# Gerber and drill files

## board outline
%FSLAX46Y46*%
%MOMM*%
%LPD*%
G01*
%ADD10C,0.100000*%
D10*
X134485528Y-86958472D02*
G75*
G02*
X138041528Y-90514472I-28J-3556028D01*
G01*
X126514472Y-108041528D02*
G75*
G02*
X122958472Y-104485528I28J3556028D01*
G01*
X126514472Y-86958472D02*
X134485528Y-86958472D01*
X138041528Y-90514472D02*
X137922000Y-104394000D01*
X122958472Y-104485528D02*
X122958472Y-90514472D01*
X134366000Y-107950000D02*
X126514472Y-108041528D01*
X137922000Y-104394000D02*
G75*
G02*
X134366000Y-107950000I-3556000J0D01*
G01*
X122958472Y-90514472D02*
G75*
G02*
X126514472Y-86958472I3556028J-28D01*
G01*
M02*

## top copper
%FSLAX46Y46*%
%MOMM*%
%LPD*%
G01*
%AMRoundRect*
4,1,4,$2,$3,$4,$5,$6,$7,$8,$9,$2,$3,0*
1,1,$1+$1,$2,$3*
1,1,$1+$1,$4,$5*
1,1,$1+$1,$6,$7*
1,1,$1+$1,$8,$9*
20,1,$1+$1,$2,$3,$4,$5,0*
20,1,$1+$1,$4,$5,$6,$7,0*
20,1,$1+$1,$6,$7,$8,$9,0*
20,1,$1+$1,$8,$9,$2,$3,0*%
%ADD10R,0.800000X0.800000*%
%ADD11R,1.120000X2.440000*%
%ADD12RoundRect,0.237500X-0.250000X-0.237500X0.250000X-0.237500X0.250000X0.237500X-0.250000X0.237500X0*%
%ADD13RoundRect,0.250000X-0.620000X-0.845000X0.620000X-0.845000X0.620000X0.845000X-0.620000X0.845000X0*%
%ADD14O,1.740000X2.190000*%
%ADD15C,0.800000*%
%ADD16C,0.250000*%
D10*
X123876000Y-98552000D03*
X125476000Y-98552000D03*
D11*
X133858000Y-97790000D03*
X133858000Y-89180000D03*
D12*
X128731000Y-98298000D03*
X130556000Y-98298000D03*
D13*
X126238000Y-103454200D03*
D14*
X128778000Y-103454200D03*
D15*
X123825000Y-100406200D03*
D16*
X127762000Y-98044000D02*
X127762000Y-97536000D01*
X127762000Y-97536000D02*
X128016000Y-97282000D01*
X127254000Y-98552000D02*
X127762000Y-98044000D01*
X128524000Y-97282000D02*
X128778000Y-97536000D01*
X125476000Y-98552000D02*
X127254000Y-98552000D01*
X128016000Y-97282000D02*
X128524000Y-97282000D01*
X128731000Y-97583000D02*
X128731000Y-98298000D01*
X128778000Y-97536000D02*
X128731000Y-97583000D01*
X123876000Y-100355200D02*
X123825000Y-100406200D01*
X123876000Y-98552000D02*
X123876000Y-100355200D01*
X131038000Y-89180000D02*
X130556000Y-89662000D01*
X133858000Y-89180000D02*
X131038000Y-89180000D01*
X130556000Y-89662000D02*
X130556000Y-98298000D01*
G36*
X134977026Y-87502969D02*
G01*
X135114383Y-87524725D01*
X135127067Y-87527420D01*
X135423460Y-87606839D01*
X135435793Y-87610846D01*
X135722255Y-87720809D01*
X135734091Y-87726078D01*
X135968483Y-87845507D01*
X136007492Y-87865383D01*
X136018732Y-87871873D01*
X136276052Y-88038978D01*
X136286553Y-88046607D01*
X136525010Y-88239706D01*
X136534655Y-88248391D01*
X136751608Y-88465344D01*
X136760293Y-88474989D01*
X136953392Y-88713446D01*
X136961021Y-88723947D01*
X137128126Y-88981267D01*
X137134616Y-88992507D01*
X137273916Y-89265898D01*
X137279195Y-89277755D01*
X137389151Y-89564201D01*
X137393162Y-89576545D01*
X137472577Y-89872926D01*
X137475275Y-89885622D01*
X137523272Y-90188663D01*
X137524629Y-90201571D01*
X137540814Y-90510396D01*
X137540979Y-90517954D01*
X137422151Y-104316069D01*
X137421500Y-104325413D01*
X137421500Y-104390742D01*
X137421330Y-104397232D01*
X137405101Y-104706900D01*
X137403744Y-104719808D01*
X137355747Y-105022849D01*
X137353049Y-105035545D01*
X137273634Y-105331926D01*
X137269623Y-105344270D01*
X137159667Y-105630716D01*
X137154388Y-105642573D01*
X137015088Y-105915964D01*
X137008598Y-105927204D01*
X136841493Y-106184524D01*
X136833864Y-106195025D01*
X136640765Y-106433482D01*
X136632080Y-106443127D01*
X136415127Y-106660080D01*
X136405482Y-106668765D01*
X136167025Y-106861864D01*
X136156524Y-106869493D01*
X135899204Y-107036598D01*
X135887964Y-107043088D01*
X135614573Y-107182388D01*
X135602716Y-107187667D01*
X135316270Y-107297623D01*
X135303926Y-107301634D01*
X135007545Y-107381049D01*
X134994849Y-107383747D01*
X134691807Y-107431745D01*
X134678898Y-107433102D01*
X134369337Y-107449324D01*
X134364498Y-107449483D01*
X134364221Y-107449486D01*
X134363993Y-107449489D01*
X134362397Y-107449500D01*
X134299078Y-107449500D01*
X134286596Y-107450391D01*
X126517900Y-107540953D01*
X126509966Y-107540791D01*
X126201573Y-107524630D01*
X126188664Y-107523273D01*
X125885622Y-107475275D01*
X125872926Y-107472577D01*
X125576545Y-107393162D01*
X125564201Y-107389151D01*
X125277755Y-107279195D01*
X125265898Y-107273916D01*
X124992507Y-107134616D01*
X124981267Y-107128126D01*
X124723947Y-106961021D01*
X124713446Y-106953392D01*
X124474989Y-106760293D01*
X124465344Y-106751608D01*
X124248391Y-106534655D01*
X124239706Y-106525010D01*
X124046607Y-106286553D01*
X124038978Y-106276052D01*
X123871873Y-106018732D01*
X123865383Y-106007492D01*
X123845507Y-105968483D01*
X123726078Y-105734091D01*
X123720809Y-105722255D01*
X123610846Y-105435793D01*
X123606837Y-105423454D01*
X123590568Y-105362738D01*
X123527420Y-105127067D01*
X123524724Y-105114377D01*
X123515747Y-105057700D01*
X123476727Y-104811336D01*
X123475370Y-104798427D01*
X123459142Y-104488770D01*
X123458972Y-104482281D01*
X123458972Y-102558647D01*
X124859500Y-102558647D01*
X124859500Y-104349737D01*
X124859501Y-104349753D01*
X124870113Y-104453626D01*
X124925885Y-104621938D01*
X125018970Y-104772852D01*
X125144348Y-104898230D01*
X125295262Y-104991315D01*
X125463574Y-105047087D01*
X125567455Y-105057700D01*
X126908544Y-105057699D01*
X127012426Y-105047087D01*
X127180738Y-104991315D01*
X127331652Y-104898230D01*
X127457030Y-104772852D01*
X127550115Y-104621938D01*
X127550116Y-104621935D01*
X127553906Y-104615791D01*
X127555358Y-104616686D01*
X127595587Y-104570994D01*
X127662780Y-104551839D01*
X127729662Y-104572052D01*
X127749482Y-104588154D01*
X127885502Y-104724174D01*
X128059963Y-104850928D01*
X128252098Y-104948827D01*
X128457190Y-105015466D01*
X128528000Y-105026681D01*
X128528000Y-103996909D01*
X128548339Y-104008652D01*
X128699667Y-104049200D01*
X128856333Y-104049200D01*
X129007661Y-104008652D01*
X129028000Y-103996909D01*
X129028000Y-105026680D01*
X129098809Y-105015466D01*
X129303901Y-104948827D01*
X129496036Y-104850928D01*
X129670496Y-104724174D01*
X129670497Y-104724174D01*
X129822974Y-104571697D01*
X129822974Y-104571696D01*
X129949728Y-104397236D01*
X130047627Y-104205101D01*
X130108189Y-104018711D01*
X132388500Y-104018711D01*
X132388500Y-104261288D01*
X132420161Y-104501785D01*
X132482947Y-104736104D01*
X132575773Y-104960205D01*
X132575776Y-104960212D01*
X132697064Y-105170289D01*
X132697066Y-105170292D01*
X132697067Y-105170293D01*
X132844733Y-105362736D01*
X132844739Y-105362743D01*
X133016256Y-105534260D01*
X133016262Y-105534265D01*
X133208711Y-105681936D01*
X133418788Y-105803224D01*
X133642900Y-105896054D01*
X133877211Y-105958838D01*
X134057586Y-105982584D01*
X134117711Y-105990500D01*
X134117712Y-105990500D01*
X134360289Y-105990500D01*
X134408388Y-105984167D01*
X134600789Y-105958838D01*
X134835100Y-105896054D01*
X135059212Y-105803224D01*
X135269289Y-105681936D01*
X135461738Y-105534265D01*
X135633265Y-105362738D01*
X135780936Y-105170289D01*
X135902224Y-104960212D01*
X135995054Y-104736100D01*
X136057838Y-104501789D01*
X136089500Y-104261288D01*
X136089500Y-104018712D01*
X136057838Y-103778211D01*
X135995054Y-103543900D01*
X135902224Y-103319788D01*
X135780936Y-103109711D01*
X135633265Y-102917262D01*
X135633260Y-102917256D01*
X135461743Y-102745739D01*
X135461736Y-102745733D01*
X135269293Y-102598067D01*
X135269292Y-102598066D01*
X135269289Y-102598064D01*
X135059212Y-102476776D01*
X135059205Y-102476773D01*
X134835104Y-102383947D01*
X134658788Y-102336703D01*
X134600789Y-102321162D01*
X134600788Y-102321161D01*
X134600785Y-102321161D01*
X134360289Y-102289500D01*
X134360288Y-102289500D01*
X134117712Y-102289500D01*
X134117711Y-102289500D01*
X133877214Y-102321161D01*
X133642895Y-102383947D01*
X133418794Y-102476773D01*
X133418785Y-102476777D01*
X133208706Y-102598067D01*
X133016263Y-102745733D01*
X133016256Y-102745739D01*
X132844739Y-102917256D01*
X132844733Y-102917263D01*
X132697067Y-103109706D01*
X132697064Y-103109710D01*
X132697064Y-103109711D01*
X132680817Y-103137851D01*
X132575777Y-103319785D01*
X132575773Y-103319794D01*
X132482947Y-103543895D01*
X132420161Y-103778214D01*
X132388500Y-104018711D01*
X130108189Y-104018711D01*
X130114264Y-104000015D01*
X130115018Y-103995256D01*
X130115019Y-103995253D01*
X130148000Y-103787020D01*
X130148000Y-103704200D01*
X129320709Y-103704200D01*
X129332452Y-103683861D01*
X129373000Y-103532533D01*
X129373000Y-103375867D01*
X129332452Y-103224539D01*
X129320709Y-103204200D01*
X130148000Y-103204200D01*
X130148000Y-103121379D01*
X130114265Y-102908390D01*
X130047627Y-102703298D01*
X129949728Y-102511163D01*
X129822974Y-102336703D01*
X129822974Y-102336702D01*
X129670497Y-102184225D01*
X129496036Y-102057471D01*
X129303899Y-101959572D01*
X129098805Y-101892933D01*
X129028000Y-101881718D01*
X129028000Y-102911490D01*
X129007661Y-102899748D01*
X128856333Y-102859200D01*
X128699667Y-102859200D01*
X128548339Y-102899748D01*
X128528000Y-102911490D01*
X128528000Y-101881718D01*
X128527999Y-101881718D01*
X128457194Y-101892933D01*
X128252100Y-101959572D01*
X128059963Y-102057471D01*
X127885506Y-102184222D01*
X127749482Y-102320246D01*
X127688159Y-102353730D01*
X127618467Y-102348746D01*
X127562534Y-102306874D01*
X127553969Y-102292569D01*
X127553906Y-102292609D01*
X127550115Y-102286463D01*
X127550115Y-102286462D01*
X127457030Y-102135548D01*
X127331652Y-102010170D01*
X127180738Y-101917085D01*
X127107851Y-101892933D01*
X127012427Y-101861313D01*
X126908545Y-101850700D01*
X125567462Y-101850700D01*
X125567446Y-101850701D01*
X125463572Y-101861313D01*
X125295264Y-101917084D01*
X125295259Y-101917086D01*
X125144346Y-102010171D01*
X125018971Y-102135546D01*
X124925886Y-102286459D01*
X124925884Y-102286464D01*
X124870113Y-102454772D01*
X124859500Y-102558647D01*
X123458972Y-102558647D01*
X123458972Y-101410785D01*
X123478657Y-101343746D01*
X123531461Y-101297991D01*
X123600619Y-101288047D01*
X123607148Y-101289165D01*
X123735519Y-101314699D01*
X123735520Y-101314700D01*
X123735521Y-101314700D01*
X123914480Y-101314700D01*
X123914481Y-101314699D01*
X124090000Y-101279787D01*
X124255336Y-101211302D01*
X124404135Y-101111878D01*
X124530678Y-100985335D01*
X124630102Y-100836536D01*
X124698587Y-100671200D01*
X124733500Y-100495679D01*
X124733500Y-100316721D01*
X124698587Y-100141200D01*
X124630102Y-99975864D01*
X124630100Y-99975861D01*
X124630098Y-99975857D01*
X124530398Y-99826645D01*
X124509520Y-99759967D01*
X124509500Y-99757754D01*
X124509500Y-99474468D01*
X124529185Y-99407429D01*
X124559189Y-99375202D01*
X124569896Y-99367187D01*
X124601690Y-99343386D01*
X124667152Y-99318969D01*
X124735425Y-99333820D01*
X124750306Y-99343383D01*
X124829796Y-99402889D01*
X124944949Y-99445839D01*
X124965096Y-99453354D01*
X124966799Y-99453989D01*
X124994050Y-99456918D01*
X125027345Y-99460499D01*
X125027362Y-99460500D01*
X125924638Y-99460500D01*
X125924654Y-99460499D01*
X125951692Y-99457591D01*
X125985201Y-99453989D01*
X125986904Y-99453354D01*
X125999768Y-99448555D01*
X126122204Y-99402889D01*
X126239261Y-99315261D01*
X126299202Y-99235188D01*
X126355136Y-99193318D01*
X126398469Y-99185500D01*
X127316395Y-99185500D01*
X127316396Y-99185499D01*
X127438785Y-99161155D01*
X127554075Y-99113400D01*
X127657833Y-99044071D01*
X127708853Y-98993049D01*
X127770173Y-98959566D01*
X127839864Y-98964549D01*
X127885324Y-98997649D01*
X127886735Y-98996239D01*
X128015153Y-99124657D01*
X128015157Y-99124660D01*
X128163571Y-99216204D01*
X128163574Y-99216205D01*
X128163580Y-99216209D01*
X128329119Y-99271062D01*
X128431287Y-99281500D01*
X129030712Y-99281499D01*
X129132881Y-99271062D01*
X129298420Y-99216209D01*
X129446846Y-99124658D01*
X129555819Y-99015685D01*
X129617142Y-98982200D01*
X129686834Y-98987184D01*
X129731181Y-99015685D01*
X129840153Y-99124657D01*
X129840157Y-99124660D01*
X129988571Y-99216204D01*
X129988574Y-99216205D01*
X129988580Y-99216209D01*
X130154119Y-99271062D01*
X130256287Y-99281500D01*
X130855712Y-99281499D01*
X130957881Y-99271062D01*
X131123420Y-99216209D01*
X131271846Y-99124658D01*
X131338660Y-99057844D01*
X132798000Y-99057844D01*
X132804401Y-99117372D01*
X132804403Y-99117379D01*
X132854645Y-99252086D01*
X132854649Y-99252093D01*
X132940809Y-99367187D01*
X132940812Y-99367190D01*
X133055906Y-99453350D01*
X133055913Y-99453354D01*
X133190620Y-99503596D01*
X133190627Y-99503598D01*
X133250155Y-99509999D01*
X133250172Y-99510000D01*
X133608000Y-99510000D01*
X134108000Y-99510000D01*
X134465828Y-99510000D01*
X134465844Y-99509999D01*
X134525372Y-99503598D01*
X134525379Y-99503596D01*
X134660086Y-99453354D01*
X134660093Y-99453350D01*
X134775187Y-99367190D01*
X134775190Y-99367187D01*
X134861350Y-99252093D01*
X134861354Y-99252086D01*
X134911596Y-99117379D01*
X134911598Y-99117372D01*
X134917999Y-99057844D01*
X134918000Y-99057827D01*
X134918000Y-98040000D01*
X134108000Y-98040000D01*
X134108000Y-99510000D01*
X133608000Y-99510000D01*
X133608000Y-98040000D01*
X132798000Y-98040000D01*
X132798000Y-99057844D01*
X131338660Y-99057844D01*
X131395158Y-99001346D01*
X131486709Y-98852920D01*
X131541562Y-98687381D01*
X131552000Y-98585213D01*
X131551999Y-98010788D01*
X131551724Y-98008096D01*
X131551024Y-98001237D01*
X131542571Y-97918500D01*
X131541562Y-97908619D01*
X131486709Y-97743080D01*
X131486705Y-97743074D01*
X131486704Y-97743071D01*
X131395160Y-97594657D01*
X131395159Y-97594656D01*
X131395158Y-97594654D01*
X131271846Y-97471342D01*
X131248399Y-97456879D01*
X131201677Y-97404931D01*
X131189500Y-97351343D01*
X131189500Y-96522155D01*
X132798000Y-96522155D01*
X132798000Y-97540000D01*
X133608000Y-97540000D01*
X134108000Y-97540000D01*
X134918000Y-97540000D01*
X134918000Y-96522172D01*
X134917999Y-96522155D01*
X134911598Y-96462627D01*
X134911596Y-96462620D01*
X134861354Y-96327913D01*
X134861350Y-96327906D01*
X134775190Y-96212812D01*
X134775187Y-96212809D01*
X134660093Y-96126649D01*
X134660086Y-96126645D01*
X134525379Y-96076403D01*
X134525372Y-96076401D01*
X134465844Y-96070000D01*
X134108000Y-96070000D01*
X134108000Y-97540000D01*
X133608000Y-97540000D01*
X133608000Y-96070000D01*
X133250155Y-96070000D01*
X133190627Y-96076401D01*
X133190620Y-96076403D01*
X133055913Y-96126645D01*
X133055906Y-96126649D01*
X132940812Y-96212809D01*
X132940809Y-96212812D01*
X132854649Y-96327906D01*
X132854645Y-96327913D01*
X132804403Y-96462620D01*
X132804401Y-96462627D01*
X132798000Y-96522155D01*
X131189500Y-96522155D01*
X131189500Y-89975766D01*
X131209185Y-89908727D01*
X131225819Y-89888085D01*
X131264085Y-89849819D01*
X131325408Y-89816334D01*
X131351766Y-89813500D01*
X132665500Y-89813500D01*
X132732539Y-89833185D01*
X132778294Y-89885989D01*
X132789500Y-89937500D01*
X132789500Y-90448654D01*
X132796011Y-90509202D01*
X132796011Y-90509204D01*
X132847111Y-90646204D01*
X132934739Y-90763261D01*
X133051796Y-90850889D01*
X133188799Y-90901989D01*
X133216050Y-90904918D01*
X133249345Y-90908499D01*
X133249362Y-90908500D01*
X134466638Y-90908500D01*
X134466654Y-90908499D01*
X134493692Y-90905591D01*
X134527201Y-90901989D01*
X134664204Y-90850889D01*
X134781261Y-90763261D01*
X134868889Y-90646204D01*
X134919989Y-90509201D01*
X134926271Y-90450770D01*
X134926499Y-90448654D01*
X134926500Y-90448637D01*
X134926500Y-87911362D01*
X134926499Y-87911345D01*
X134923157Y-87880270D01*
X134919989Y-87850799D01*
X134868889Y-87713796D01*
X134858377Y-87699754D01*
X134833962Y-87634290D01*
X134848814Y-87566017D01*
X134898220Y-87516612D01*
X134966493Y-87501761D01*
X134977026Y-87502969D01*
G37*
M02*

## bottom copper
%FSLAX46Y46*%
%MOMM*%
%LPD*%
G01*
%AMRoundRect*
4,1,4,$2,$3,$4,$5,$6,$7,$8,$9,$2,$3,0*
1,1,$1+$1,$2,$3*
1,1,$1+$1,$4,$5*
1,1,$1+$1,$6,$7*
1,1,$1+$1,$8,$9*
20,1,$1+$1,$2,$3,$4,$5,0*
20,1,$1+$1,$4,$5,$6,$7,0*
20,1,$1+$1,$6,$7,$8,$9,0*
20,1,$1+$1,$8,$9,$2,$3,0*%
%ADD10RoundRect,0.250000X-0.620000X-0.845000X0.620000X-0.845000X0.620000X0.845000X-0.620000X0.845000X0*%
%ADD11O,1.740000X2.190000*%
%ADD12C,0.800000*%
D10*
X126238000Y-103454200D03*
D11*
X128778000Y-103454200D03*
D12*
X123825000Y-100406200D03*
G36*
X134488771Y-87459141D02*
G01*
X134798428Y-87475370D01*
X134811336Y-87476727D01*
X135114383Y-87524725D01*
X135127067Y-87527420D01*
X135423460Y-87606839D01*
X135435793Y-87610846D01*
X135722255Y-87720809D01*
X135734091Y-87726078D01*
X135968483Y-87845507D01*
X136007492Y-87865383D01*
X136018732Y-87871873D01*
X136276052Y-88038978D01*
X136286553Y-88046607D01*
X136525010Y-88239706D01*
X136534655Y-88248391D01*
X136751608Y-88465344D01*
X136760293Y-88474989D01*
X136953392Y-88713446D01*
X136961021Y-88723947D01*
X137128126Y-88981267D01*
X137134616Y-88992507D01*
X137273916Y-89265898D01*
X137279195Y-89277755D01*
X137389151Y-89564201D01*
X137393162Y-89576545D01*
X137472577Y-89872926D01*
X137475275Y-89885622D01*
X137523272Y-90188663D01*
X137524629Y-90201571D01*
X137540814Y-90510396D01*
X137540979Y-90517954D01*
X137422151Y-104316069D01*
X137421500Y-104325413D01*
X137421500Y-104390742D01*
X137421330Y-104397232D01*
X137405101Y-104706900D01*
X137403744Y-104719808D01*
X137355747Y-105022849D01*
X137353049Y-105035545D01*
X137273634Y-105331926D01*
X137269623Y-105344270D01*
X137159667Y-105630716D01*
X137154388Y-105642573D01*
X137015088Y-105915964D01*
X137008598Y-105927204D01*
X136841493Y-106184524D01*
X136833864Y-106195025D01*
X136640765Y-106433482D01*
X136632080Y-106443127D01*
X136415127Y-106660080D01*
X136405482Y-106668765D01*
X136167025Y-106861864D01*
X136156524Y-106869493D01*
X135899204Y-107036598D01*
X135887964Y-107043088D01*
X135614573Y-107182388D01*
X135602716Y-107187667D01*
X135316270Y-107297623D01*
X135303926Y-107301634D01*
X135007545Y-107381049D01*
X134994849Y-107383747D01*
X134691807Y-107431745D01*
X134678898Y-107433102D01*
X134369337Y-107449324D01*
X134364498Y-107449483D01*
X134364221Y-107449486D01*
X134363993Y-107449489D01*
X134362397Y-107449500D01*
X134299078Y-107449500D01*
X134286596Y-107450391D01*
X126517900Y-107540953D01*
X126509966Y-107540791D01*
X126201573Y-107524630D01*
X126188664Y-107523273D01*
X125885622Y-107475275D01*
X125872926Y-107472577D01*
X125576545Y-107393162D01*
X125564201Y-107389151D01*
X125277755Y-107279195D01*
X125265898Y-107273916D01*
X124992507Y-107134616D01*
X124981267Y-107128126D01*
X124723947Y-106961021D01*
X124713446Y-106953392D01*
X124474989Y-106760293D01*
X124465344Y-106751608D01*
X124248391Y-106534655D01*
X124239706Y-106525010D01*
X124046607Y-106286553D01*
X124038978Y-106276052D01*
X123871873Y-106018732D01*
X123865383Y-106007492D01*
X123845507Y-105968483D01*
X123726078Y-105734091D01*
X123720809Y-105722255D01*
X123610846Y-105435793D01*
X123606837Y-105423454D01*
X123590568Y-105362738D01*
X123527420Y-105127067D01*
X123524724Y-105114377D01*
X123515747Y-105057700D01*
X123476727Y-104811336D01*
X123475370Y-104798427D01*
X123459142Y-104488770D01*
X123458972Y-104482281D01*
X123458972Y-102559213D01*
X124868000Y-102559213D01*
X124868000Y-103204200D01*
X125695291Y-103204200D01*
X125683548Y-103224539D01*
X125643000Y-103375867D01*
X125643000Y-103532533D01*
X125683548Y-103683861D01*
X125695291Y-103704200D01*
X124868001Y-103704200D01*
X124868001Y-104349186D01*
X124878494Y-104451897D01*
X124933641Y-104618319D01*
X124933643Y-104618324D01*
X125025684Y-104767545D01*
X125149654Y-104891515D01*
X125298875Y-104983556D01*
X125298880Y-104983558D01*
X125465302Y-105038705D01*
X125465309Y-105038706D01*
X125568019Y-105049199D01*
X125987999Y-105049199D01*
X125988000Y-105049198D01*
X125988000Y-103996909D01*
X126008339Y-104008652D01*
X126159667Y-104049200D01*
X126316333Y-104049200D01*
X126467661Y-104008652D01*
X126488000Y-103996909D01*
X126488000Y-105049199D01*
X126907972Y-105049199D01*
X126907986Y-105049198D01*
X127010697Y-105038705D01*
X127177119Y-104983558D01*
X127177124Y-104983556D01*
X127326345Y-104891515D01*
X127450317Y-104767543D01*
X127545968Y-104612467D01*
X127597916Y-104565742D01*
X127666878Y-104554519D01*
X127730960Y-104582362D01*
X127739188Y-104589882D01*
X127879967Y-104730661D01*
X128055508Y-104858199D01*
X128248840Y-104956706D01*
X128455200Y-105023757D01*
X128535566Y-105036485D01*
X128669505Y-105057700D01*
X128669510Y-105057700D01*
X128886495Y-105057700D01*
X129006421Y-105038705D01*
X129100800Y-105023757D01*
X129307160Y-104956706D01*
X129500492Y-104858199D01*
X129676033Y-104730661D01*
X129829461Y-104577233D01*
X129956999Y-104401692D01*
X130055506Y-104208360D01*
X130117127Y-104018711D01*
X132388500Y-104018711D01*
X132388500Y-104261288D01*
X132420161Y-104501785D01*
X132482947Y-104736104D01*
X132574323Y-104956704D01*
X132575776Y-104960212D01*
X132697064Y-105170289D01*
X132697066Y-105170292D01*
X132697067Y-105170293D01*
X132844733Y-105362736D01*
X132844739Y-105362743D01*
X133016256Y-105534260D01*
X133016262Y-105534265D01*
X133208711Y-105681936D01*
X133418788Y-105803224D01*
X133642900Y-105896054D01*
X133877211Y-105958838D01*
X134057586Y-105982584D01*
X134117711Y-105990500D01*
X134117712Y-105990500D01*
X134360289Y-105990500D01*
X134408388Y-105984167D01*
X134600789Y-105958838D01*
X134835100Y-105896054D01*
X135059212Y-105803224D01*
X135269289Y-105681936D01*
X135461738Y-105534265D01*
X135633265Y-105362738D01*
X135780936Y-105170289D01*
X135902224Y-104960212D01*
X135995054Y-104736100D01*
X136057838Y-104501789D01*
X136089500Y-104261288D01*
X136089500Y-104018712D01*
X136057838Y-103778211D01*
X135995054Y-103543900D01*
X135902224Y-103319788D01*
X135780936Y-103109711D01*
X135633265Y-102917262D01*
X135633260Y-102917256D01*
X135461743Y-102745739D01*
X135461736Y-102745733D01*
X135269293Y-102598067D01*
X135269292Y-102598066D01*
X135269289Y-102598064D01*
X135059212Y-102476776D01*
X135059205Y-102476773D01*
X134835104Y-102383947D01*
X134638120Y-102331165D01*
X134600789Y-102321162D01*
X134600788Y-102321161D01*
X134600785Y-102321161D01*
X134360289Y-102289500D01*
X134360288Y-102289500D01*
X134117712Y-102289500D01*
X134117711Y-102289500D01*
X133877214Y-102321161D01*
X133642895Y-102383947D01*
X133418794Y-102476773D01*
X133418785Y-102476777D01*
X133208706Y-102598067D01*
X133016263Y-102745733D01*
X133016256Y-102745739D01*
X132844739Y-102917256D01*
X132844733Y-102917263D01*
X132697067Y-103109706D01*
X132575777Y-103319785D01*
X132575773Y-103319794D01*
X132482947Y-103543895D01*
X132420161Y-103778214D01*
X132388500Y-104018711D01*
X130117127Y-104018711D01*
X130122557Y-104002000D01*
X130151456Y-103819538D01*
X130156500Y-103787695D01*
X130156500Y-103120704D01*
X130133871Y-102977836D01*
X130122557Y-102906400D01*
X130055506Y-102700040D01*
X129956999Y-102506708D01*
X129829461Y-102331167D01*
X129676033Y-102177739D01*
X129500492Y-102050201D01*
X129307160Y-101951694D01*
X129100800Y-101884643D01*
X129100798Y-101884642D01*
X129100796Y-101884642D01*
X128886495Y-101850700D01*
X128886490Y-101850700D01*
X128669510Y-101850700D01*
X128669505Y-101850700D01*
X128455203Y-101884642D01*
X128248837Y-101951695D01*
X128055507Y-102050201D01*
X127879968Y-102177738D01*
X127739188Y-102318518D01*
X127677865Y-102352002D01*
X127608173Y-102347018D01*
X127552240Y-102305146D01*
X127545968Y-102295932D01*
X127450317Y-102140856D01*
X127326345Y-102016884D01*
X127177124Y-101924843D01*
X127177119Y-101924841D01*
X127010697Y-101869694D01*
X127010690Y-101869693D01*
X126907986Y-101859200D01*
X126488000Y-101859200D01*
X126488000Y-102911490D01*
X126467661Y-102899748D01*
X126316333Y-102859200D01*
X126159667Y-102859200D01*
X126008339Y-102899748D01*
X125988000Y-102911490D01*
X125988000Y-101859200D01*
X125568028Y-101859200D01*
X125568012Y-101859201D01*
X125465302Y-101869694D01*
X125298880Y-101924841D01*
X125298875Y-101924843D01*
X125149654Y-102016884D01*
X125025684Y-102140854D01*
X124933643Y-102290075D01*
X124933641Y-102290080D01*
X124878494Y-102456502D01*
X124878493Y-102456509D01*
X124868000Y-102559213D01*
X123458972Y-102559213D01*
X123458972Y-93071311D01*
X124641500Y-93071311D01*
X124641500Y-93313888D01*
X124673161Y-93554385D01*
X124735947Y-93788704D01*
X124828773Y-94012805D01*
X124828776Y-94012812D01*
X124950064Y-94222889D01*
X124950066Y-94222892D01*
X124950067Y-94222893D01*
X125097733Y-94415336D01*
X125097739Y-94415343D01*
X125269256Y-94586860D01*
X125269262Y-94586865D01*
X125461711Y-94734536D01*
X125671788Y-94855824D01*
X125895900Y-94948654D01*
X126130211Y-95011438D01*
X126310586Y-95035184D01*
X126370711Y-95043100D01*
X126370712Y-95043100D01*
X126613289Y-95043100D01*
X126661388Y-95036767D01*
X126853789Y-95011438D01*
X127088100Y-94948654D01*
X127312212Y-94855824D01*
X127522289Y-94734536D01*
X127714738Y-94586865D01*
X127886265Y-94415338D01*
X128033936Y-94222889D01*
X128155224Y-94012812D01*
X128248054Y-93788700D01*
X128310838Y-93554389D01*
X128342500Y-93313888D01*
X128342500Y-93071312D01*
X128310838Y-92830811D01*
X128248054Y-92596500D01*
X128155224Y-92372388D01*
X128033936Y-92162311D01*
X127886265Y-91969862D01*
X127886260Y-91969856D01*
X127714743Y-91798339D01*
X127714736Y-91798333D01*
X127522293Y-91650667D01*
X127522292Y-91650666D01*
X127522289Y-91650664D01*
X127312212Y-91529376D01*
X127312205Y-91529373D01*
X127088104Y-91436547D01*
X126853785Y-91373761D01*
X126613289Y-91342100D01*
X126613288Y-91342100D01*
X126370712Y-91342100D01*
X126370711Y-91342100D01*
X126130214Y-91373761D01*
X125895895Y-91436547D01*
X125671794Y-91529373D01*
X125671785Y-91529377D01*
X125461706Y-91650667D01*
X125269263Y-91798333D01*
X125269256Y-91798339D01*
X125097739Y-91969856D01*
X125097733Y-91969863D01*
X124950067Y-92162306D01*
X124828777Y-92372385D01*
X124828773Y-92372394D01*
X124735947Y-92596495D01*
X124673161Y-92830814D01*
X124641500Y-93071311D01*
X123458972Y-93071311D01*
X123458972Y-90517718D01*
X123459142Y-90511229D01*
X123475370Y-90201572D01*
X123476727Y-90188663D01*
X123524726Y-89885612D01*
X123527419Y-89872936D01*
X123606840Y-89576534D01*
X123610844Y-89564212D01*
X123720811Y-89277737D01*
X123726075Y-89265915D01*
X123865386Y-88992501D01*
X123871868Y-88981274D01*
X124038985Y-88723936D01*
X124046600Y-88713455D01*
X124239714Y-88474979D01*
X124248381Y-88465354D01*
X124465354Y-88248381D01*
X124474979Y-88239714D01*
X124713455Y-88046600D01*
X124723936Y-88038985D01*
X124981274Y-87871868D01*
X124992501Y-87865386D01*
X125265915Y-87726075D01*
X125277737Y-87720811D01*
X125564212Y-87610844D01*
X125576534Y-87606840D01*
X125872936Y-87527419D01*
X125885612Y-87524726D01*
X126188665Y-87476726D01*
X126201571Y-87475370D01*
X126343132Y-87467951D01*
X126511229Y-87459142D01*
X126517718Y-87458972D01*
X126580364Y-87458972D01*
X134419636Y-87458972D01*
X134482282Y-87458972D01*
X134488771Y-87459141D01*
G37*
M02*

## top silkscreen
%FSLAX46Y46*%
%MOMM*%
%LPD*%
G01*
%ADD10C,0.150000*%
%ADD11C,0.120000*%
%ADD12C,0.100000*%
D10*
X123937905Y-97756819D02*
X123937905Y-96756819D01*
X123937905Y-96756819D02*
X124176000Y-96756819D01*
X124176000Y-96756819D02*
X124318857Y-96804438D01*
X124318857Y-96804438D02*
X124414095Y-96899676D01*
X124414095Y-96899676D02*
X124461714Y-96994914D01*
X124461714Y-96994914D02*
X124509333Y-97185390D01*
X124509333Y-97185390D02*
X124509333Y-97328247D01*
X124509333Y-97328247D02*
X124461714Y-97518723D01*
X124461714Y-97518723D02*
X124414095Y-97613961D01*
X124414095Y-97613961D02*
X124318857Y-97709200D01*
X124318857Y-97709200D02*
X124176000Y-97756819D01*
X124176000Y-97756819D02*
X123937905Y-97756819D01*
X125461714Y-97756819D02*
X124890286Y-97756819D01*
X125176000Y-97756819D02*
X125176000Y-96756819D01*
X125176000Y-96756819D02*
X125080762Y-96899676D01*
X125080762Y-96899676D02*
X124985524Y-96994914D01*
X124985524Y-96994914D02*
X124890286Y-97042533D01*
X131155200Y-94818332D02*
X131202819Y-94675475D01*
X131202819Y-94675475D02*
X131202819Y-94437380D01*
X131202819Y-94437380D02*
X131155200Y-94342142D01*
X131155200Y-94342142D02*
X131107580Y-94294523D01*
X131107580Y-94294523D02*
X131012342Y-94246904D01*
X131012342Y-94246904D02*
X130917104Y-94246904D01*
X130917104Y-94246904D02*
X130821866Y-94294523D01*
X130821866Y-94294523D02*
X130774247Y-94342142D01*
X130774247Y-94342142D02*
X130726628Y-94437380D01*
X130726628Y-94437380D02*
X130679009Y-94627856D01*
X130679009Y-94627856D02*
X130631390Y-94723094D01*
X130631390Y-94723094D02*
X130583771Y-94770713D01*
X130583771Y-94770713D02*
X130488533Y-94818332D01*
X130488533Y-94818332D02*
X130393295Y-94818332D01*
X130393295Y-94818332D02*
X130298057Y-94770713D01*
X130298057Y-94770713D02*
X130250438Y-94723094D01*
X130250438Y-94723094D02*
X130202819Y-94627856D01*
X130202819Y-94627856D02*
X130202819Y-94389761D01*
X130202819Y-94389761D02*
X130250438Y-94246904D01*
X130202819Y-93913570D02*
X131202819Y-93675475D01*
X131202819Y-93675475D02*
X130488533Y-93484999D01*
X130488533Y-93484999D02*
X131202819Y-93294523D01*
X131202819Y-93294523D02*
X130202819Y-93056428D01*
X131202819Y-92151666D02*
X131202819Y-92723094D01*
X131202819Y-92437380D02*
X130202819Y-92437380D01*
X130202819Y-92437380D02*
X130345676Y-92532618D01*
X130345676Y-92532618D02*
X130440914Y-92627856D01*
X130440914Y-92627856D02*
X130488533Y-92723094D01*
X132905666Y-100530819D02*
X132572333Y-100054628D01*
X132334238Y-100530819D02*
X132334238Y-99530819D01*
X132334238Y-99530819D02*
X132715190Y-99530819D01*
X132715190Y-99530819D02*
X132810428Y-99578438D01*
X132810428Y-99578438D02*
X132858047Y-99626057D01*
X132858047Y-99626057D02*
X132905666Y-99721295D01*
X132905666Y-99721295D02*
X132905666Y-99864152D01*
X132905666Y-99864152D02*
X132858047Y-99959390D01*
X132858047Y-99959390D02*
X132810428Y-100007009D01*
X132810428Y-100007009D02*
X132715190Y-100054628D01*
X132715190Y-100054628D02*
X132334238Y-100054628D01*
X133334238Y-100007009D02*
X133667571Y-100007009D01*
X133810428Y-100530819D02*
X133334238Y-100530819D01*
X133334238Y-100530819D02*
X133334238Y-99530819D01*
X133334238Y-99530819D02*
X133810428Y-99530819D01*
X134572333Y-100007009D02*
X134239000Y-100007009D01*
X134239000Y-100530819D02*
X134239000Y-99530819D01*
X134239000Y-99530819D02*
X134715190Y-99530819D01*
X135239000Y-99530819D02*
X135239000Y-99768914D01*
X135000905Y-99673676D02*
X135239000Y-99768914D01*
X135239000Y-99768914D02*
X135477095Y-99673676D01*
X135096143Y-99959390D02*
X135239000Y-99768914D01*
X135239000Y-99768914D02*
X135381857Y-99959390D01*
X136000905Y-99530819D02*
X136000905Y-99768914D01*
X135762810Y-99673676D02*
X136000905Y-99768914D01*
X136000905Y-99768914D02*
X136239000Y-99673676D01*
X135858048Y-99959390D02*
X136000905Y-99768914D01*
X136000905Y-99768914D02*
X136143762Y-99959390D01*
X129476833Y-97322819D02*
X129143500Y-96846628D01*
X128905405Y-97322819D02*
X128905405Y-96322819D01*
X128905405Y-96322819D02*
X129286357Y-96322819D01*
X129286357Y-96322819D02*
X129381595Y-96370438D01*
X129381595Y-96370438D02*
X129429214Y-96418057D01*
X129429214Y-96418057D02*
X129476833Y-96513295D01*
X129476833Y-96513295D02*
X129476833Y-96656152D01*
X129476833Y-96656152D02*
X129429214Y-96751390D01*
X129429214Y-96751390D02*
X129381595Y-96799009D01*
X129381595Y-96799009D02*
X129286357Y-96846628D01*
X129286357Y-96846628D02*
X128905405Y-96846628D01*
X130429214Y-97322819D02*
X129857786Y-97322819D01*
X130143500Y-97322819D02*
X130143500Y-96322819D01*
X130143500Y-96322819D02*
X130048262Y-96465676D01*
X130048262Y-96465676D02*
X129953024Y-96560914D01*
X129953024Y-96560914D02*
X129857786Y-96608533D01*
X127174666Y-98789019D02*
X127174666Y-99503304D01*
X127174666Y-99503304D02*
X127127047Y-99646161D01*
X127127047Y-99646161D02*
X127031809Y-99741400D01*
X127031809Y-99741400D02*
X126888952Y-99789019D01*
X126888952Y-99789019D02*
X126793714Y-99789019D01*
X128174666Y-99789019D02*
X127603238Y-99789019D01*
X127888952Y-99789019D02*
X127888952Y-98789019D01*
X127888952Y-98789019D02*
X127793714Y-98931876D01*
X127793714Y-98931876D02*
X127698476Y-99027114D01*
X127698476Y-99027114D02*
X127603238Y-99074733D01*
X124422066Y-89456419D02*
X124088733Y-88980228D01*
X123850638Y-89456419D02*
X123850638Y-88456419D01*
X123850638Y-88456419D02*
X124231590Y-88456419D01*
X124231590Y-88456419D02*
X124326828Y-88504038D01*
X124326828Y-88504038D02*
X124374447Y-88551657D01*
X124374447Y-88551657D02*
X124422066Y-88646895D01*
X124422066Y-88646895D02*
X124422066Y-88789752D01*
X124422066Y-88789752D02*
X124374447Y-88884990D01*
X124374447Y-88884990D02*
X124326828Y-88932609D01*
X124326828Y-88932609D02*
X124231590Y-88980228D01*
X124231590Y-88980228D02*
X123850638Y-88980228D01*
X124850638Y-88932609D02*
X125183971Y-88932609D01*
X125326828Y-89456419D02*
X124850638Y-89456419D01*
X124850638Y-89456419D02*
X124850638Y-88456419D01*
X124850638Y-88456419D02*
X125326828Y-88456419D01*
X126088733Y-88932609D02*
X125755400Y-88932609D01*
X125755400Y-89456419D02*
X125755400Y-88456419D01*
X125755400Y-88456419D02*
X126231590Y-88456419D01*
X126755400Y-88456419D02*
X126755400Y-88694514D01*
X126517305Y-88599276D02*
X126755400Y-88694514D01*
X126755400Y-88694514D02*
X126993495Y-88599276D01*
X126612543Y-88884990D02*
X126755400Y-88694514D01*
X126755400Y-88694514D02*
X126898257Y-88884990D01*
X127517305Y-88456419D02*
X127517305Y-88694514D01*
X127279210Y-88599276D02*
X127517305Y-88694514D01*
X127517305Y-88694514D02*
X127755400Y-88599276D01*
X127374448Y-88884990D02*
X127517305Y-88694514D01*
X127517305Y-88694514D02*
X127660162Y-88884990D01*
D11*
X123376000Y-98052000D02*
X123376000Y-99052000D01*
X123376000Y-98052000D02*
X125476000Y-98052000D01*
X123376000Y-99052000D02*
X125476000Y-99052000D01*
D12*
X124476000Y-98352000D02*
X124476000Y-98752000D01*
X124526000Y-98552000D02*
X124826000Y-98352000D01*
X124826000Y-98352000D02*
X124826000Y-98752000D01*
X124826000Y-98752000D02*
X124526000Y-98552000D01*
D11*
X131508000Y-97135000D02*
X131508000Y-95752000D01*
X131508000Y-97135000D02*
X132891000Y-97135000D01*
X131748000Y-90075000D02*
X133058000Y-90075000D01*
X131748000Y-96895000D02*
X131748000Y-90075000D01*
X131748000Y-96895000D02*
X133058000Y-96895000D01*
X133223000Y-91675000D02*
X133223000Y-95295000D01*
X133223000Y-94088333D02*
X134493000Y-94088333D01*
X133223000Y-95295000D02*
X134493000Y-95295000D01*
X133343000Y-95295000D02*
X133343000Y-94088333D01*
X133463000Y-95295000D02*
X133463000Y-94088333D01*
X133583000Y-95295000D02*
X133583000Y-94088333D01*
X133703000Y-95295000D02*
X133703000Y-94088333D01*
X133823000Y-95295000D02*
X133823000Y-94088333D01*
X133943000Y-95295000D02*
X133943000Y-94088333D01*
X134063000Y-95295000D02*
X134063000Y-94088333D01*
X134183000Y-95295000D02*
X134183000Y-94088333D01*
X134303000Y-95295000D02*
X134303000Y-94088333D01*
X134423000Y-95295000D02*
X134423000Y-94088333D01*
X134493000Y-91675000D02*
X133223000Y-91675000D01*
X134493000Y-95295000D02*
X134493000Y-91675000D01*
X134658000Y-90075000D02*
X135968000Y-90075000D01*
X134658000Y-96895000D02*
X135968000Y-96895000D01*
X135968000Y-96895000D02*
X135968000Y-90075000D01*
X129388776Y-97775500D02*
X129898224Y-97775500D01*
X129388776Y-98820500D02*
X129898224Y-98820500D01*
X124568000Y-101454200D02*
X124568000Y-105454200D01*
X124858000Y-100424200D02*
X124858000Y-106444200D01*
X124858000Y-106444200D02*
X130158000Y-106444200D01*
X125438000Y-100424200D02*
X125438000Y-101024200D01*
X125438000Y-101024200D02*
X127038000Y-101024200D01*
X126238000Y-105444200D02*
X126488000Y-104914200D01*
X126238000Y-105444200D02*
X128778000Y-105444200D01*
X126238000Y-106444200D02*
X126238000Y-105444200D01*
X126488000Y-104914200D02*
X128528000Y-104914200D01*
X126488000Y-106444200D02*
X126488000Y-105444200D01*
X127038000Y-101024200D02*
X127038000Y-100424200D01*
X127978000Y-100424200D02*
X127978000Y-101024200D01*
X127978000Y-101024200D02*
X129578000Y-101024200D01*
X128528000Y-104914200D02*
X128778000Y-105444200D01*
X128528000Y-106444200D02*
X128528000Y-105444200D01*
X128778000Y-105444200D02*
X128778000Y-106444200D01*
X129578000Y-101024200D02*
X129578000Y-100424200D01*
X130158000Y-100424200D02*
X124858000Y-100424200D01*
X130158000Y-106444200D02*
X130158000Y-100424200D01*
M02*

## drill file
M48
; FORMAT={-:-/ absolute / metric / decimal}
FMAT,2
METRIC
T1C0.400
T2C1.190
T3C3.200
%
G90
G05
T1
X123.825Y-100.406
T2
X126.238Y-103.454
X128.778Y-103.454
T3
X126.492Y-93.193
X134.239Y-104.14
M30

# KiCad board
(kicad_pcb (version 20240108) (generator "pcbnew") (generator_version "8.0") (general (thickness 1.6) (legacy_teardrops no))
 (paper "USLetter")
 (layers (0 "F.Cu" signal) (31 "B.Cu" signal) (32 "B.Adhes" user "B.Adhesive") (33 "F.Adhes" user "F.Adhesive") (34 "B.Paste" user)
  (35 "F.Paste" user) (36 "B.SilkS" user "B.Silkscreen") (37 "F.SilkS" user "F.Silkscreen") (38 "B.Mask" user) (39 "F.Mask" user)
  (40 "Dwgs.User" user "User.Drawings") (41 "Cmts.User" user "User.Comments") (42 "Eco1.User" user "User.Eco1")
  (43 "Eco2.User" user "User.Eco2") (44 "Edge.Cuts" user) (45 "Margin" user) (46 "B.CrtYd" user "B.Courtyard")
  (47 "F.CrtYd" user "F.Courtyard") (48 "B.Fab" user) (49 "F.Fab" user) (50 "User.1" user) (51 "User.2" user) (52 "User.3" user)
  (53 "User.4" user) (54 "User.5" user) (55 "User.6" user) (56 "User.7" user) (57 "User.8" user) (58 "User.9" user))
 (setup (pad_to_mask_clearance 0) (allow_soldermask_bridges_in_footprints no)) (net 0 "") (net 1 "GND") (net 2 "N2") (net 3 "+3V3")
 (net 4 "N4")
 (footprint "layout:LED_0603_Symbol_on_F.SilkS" (layer "F.Cu") (at 124.676 98.552)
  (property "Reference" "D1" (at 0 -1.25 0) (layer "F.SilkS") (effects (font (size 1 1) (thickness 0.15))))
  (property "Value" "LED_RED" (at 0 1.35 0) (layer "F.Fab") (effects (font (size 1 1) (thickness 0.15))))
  (fp_line (start -1.3 -0.5) (end -1.3 0.5) (stroke (width 0.12) (type solid)) (layer "F.SilkS"))
  (fp_line (start -1.3 -0.5) (end 0.8 -0.5) (stroke (width 0.12) (type solid)) (layer "F.SilkS"))
  (fp_line (start -1.3 0.5) (end 0.8 0.5) (stroke (width 0.12) (type solid)) (layer "F.SilkS"))
  (fp_line (start -0.2 -0.2) (end -0.2 0.2) (stroke (width 0.1) (type solid)) (layer "F.SilkS"))
  (fp_line (start -0.15 0) (end 0.15 -0.2) (stroke (width 0.1) (type solid)) (layer "F.SilkS"))
  (fp_line (start 0.15 -0.2) (end 0.15 0.2) (stroke (width 0.1) (type solid)) (layer "F.SilkS"))
  (fp_line (start 0.15 0.2) (end -0.15 0) (stroke (width 0.1) (type solid)) (layer "F.SilkS"))
  (pad "1" smd rect (at -0.8 0 180) (size 0.8 0.8) (layers "F.Cu" "F.Paste" "F.Mask") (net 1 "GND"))
  (pad "2" smd rect (at 0.8 0 180) (size 0.8 0.8) (layers "F.Cu" "F.Paste" "F.Mask") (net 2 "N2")))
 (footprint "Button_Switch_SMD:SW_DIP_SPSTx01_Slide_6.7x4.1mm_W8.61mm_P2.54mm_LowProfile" (layer "F.Cu") (at 133.858 93.485 90)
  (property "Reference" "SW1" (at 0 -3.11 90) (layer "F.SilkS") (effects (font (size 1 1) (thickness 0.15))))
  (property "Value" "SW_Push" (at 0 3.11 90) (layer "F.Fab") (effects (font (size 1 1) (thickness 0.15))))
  (fp_line (start -3.65 -2.35) (end -2.267 -2.35) (stroke (width 0.12) (type solid)) (layer "F.SilkS"))
  (fp_line (start -3.65 -2.35) (end -3.65 -0.967) (stroke (width 0.12) (type solid)) (layer "F.SilkS"))
  (fp_line (start 3.41 -2.11) (end 3.41 -0.8) (stroke (width 0.12) (type solid)) (layer "F.SilkS"))
  (fp_line (start -3.41 -2.11) (end 3.41 -2.11) (stroke (width 0.12) (type solid)) (layer "F.SilkS"))
  (fp_line (start -3.41 -2.11) (end -3.41 -0.8) (stroke (width 0.12) (type solid)) (layer "F.SilkS"))
  (fp_line (start 1.81 -0.635) (end -1.81 -0.635) (stroke (width 0.12) (type solid)) (layer "F.SilkS"))
  (fp_line (start -0.603333 -0.635) (end -0.603333 0.635) (stroke (width 0.12) (type solid)) (layer "F.SilkS"))
  (fp_line (start -1.81 -0.635) (end -1.81 0.635) (stroke (width 0.12) (type solid)) (layer "F.SilkS"))
  (fp_line (start -1.81 -0.515) (end -0.603333 -0.515) (stroke (width 0.12) (type solid)) (layer "F.SilkS"))
  (fp_line (start -1.81 -0.395) (end -0.603333 -0.395) (stroke (width 0.12) (type solid)) (layer "F.SilkS"))
  (fp_line (start -1.81 -0.275) (end -0.603333 -0.275) (stroke (width 0.12) (type solid)) (layer "F.SilkS"))
  (fp_line (start -1.81 -0.155) (end -0.603333 -0.155) (stroke (width 0.12) (type solid)) (layer "F.SilkS"))
  (fp_line (start -1.81 -0.035) (end -0.603333 -0.035) (stroke (width 0.12) (type solid)) (layer "F.SilkS"))
  (fp_line (start -1.81 0.085) (end -0.603333 0.085) (stroke (width 0.12) (type solid)) (layer "F.SilkS"))
  (fp_line (start -1.81 0.205) (end -0.603333 0.205) (stroke (width 0.12) (type solid)) (layer "F.SilkS"))
  (fp_line (start -1.81 0.325) (end -0.603333 0.325) (stroke (width 0.12) (type solid)) (layer "F.SilkS"))
  (fp_line (start -1.81 0.445) (end -0.603333 0.445) (stroke (width 0.12) (type solid)) (layer "F.SilkS"))
  (fp_line (start -1.81 0.565) (end -0.603333 0.565) (stroke (width 0.12) (type solid)) (layer "F.SilkS"))
  (fp_line (start 1.81 0.635) (end 1.81 -0.635) (stroke (width 0.12) (type solid)) (layer "F.SilkS"))
  (fp_line (start -1.81 0.635) (end 1.81 0.635) (stroke (width 0.12) (type solid)) (layer "F.SilkS"))
  (fp_line (start 3.41 0.8) (end 3.41 2.11) (stroke (width 0.12) (type solid)) (layer "F.SilkS"))
  (fp_line (start -3.41 0.8) (end -3.41 2.11) (stroke (width 0.12) (type solid)) (layer "F.SilkS"))
  (fp_line (start -3.41 2.11) (end 3.41 2.11) (stroke (width 0.12) (type solid)) (layer "F.SilkS"))
  (pad "1" smd rect (at -4.305 0 90) (size 2.44 1.12) (layers "F.Cu" "F.Paste" "F.Mask") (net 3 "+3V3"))
  (pad "2" smd rect (at 4.305 0 90) (size 2.44 1.12) (layers "F.Cu" "F.Paste" "F.Mask") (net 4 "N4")))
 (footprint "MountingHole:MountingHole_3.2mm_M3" (layer "F.Cu") (at 134.239 104.14)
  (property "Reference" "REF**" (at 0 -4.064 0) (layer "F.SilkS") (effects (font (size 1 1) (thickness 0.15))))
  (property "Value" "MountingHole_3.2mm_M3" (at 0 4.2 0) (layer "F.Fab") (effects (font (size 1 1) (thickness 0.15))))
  (pad "" np_thru_hole circle (at 0 0) (size 3.2 3.2) (drill 3.2) (layers "*.Cu" "*.Mask")))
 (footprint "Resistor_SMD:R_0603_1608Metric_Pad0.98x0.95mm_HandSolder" (layer "F.Cu") (at 129.6435 98.298)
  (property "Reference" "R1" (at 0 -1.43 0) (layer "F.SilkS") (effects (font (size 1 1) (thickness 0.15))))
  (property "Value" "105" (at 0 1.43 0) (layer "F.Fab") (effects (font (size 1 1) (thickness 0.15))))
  (fp_line (start -0.254724 -0.5225) (end 0.254724 -0.5225) (stroke (width 0.12) (type solid)) (layer "F.SilkS"))
  (fp_line (start -0.254724 0.5225) (end 0.254724 0.5225) (stroke (width 0.12) (type solid)) (layer "F.SilkS"))
  (pad "1" smd roundrect (at -0.9125 0) (size 0.975 0.95) (layers "F.Cu" "F.Paste" "F.Mask") (roundrect_rratio 0.25) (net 2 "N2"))
  (pad "2" smd roundrect (at 0.9125 0) (size 0.975 0.95) (layers "F.Cu" "F.Paste" "F.Mask") (roundrect_rratio 0.25) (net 4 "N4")))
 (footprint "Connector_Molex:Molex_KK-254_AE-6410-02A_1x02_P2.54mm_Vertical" (layer "F.Cu") (at 126.238 103.4542)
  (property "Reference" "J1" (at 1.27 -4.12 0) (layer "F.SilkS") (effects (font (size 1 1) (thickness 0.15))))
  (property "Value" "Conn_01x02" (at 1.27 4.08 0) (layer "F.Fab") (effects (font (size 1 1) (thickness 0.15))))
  (fp_line (start -1.67 -2) (end -1.67 2) (stroke (width 0.12) (type solid)) (layer "F.SilkS"))
  (fp_line (start -1.38 -3.03) (end -1.38 2.99) (stroke (width 0.12) (type solid)) (layer "F.SilkS"))
  (fp_line (start -1.38 2.99) (end 3.92 2.99) (stroke (width 0.12) (type solid)) (layer "F.SilkS"))
  (fp_line (start -0.8 -3.03) (end -0.8 -2.43) (stroke (width 0.12) (type solid)) (layer "F.SilkS"))
  (fp_line (start -0.8 -2.43) (end 0.8 -2.43) (stroke (width 0.12) (type solid)) (layer "F.SilkS"))
  (fp_line (start 0 1.99) (end 0.25 1.46) (stroke (width 0.12) (type solid)) (layer "F.SilkS"))
  (fp_line (start 0 1.99) (end 2.54 1.99) (stroke (width 0.12) (type solid)) (layer "F.SilkS"))
  (fp_line (start 0 2.99) (end 0 1.99) (stroke (width 0.12) (type solid)) (layer "F.SilkS"))
  (fp_line (start 0.25 1.46) (end 2.29 1.46) (stroke (width 0.12) (type solid)) (layer "F.SilkS"))
  (fp_line (start 0.25 2.99) (end 0.25 1.99) (stroke (width 0.12) (type solid)) (layer "F.SilkS"))
  (fp_line (start 0.8 -2.43) (end 0.8 -3.03) (stroke (width 0.12) (type solid)) (layer "F.SilkS"))
  (fp_line (start 1.74 -3.03) (end 1.74 -2.43) (stroke (width 0.12) (type solid)) (layer "F.SilkS"))
  (fp_line (start 1.74 -2.43) (end 3.34 -2.43) (stroke (width 0.12) (type solid)) (layer "F.SilkS"))
  (fp_line (start 2.29 1.46) (end 2.54 1.99) (stroke (width 0.12) (type solid)) (layer "F.SilkS"))
  (fp_line (start 2.29 2.99) (end 2.29 1.99) (stroke (width 0.12) (type solid)) (layer "F.SilkS"))
  (fp_line (start 2.54 1.99) (end 2.54 2.99) (stroke (width 0.12) (type solid)) (layer "F.SilkS"))
  (fp_line (start 3.34 -2.43) (end 3.34 -3.03) (stroke (width 0.12) (type solid)) (layer "F.SilkS"))
  (fp_line (start 3.92 -3.03) (end -1.38 -3.03) (stroke (width 0.12) (type solid)) (layer "F.SilkS"))
  (fp_line (start 3.92 2.99) (end 3.92 -3.03) (stroke (width 0.12) (type solid)) (layer "F.SilkS"))
  (pad "1" thru_hole roundrect (at 0 0) (size 1.74 2.19) (drill 1.19) (layers "*.Cu" "*.Mask") (remove_unused_layers no)
   (roundrect_rratio 0.143678) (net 1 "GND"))
  (pad "2" thru_hole oval (at 2.54 0) (size 1.74 2.19) (drill 1.19) (layers "*.Cu" "*.Mask") (remove_unused_layers no) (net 3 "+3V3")))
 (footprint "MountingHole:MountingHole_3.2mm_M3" (layer "F.Cu") (at 126.492 93.1926)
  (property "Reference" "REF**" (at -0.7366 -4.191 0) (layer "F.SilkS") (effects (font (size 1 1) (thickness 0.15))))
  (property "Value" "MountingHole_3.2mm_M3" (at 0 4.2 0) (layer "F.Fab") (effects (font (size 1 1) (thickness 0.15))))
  (pad "" np_thru_hole circle (at 0 0) (size 3.2 3.2) (drill 3.2) (layers "*.Cu" "*.Mask")))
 (gr_arc (start 134.485528 86.958472) (mid 137 88) (end 138.041528 90.514472) (stroke (width 0.1) (type default)) (layer "Edge.Cuts"))
 (gr_arc (start 126.514472 108.041528) (mid 124 107) (end 122.958472 104.485528) (stroke (width 0.1) (type default)) (layer "Edge.Cuts"))
 (gr_line (start 126.514472 86.958472) (end 134.485528 86.958472) (stroke (width 0.1) (type default)) (layer "Edge.Cuts"))
 (gr_line (start 138.041528 90.514472) (end 137.922 104.394) (stroke (width 0.1) (type default)) (layer "Edge.Cuts"))
 (gr_line (start 122.958472 104.485528) (end 122.958472 90.514472) (stroke (width 0.1) (type default)) (layer "Edge.Cuts"))
 (gr_line (start 134.366 107.95) (end 126.514472 108.041528) (stroke (width 0.1) (type default)) (layer "Edge.Cuts"))
 (gr_arc (start 137.922 104.394) (mid 136.880472 106.908472) (end 134.366 107.95) (stroke (width 0.1) (type default)) (layer "Edge.Cuts"))
 (gr_arc (start 122.958472 90.514472) (mid 124 88) (end 126.514472 86.958472) (stroke (width 0.1) (type default)) (layer "Edge.Cuts"))
 (segment (start 127.762 98.044) (end 127.762 97.536) (width 0.25) (layer "F.Cu") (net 2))
 (segment (start 127.762 97.536) (end 128.016 97.282) (width 0.25) (layer "F.Cu") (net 2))
 (segment (start 127.254 98.552) (end 127.762 98.044) (width 0.25) (layer "F.Cu") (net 2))
 (segment (start 128.524 97.282) (end 128.778 97.536) (width 0.25) (layer "F.Cu") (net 2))
 (segment (start 125.476 98.552) (end 127.254 98.552) (width 0.25) (layer "F.Cu") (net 2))
 (segment (start 128.016 97.282) (end 128.524 97.282) (width 0.25) (layer "F.Cu") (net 2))
 (segment (start 128.731 97.583) (end 128.731 98.298) (width 0.25) (layer "F.Cu") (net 2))
 (segment (start 128.778 97.536) (end 128.731 97.583) (width 0.25) (layer "F.Cu") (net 2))
 (segment (start 123.876 100.3552) (end 123.825 100.4062) (width 0.25) (layer "F.Cu") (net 1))
 (segment (start 123.876 98.552) (end 123.876 100.3552) (width 0.25) (layer "F.Cu") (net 1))
 (via (at 123.825 100.4062) (size 0.8) (drill 0.4) (layers "F.Cu" "B.Cu") (free yes) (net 1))
 (segment (start 131.038 89.18) (end 130.556 89.662) (width 0.25) (layer "F.Cu") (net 4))
 (segment (start 133.858 89.18) (end 131.038 89.18) (width 0.25) (layer "F.Cu") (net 4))
 (segment (start 130.556 89.662) (end 130.556 98.298) (width 0.25) (layer "F.Cu") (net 4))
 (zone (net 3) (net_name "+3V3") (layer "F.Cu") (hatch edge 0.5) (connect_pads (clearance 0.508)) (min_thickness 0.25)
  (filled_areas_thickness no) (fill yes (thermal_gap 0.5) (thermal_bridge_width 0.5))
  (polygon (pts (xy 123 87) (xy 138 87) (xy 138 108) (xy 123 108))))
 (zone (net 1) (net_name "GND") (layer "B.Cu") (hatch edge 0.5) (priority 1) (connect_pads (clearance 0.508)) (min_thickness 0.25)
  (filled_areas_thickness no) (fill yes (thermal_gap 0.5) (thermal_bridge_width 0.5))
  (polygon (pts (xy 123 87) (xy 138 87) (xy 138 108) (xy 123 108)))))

